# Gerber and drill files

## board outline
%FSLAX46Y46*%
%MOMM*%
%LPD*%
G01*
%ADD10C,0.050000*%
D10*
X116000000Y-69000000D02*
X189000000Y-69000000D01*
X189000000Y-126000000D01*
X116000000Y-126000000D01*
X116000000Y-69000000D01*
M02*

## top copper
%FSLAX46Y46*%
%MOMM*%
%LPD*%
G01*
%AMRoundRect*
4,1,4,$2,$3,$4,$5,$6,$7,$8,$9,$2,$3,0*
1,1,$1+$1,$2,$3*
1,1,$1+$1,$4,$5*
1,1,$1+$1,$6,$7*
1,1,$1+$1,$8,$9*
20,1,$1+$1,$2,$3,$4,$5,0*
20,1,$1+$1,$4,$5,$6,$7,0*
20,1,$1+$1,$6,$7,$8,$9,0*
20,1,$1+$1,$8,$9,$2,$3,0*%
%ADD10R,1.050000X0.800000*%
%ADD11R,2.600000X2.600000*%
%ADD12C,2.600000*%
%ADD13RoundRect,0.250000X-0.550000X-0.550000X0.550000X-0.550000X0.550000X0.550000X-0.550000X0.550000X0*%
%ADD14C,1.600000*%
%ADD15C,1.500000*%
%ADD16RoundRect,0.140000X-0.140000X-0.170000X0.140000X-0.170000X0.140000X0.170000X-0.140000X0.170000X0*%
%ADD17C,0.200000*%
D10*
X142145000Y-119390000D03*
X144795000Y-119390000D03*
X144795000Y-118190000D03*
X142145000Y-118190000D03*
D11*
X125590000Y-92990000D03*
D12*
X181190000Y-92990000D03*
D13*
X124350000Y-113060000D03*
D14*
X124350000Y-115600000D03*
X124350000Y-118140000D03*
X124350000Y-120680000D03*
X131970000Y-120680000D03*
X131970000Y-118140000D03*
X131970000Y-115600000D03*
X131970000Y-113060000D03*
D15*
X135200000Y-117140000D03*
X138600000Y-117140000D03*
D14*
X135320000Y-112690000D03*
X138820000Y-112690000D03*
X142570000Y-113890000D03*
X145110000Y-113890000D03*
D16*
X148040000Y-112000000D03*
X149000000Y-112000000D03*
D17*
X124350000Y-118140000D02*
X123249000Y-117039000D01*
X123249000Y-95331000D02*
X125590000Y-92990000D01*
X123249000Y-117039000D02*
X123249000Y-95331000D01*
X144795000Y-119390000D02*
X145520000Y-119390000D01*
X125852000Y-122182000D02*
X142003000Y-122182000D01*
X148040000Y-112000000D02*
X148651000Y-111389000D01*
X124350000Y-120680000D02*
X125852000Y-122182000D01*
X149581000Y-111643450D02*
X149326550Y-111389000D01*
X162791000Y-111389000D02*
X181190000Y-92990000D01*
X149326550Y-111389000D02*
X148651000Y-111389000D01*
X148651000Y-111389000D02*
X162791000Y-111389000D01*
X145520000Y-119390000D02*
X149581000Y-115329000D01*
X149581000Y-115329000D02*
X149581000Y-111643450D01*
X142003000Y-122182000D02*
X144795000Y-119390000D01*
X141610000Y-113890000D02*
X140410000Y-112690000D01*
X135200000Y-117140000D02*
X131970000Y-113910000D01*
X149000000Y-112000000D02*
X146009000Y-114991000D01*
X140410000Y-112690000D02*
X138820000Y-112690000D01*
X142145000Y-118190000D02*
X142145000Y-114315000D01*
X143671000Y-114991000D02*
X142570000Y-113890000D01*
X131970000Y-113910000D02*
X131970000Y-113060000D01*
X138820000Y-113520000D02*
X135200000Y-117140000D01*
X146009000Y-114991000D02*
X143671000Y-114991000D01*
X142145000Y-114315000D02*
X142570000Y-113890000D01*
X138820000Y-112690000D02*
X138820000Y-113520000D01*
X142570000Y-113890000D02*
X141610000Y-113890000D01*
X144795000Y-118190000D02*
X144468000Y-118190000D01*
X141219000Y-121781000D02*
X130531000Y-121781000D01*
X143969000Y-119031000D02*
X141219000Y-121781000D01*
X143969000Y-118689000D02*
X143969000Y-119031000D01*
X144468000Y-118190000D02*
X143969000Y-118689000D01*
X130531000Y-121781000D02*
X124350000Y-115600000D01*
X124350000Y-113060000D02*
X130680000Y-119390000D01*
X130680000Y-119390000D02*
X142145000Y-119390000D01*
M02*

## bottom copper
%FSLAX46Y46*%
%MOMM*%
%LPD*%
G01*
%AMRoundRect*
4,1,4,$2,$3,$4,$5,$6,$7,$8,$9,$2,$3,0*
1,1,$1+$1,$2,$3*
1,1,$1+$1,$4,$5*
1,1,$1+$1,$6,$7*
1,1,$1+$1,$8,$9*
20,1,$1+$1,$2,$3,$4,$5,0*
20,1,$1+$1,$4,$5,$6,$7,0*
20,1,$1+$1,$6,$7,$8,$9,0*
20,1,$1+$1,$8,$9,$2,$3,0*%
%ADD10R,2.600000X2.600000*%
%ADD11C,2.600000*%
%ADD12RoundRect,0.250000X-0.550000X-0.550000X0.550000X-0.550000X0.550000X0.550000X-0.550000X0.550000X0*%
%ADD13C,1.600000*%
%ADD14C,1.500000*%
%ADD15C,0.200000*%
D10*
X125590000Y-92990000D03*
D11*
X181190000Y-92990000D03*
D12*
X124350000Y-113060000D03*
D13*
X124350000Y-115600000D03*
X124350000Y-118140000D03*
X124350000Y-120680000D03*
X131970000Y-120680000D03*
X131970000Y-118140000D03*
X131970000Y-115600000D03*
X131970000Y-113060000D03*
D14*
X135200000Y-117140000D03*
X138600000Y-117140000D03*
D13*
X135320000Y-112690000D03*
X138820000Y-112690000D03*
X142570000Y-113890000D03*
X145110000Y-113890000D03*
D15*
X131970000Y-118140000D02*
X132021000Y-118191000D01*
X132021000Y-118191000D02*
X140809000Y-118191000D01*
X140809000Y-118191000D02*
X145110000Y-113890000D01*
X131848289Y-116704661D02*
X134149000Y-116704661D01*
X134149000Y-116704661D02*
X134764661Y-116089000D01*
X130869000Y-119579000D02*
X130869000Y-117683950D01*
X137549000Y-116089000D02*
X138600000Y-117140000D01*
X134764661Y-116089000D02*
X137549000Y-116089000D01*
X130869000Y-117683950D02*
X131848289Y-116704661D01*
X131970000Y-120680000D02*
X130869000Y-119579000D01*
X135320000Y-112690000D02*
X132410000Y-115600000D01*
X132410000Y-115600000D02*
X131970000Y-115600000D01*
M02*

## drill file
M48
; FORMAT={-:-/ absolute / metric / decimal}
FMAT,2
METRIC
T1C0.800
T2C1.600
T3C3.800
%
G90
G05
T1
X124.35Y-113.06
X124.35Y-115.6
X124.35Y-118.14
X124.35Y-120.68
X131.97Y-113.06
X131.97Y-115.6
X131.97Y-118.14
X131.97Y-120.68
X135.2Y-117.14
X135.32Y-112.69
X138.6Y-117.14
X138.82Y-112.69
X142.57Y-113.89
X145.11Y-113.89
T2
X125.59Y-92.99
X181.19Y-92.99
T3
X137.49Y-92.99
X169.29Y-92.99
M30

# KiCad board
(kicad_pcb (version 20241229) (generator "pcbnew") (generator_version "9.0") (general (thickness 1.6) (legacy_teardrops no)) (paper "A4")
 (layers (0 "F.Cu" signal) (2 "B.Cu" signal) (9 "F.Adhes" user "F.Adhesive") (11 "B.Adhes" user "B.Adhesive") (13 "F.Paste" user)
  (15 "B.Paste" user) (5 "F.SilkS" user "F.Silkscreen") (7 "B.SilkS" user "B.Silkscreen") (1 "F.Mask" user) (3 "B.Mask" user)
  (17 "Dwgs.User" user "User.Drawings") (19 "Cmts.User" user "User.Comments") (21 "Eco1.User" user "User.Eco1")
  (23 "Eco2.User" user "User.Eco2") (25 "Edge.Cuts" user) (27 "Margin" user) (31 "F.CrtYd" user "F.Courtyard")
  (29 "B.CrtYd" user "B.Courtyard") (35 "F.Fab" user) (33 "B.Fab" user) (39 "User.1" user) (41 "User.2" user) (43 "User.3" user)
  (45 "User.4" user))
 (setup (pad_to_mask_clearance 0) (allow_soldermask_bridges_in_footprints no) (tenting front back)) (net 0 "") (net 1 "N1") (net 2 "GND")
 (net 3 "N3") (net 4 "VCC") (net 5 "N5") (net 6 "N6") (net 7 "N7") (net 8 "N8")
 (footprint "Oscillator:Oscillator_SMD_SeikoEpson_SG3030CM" (layer "F.Cu") (at 143.47 118.79)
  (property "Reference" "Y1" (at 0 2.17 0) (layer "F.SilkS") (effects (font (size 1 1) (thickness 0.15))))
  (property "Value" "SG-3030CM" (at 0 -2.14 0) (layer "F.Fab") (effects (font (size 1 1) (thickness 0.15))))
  (pad "1" smd rect (at -1.325 0.6) (size 1.05 0.8) (layers "F.Cu" "F.Mask" "F.Paste") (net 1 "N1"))
  (pad "2" smd rect (at 1.325 0.6) (size 1.05 0.8) (layers "F.Cu" "F.Mask" "F.Paste") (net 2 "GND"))
  (pad "3" smd rect (at 1.325 -0.6) (size 1.05 0.8) (layers "F.Cu" "F.Mask" "F.Paste") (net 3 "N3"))
  (pad "4" smd rect (at -1.325 -0.6) (size 1.05 0.8) (layers "F.Cu" "F.Mask" "F.Paste") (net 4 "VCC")))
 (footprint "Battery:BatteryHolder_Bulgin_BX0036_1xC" (layer "F.Cu") (at 125.59 92.99)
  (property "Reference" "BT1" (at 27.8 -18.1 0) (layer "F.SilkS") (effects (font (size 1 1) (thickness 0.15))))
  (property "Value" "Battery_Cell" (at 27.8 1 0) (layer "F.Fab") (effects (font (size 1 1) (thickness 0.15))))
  (pad "" np_thru_hole circle (at 11.9 0) (size 3.8 3.8) (drill 3.8) (layers "*.Cu" "*.Mask"))
  (pad "" np_thru_hole circle (at 43.7 0) (size 3.8 3.8) (drill 3.8) (layers "*.Cu" "*.Mask"))
  (pad "1" thru_hole rect (at 0 0) (size 2.6 2.6) (drill 1.6) (layers "*.Cu" "*.Mask") (remove_unused_layers no) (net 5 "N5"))
  (pad "2" thru_hole circle (at 55.6 0) (size 2.6 2.6) (drill 1.6) (layers "*.Cu" "*.Mask") (remove_unused_layers no) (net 2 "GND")))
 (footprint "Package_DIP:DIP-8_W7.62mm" (layer "F.Cu") (at 124.35 113.06)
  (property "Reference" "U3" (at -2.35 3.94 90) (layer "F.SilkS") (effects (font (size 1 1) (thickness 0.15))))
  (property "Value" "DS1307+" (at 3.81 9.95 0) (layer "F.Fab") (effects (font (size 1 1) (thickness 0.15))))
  (pad "1" thru_hole roundrect (at 0 0) (size 1.6 1.6) (drill 0.8) (layers "*.Cu" "*.Mask") (remove_unused_layers no)
   (roundrect_rratio 0.15625) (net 1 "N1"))
  (pad "2" thru_hole circle (at 0 2.54) (size 1.6 1.6) (drill 0.8) (layers "*.Cu" "*.Mask") (remove_unused_layers no) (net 3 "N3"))
  (pad "3" thru_hole circle (at 0 5.08) (size 1.6 1.6) (drill 0.8) (layers "*.Cu" "*.Mask") (remove_unused_layers no) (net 5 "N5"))
  (pad "4" thru_hole circle (at 0 7.62) (size 1.6 1.6) (drill 0.8) (layers "*.Cu" "*.Mask") (remove_unused_layers no) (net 2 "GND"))
  (pad "5" thru_hole circle (at 7.62 7.62) (size 1.6 1.6) (drill 0.8) (layers "*.Cu" "*.Mask") (remove_unused_layers no) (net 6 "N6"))
  (pad "6" thru_hole circle (at 7.62 5.08) (size 1.6 1.6) (drill 0.8) (layers "*.Cu" "*.Mask") (remove_unused_layers no) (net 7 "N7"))
  (pad "7" thru_hole circle (at 7.62 2.54) (size 1.6 1.6) (drill 0.8) (layers "*.Cu" "*.Mask") (remove_unused_layers no) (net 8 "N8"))
  (pad "8" thru_hole circle (at 7.62 0) (size 1.6 1.6) (drill 0.8) (layers "*.Cu" "*.Mask") (remove_unused_layers no) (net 4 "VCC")))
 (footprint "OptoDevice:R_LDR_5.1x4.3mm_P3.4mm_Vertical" (layer "F.Cu") (at 135.2 117.14)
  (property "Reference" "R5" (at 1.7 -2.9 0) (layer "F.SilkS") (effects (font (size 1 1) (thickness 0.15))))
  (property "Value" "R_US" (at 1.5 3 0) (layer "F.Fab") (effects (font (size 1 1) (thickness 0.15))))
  (pad "1" thru_hole circle (at 0 0) (size 1.5 1.5) (drill 0.8) (layers "*.Cu" "*.Mask") (remove_unused_layers no) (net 4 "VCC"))
  (pad "2" thru_hole circle (at 3.4 0) (size 1.5 1.5) (drill 0.8) (layers "*.Cu" "*.Mask") (remove_unused_layers no) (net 6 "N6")))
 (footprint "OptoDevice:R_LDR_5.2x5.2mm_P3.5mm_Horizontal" (layer "F.Cu") (at 135.32 112.69)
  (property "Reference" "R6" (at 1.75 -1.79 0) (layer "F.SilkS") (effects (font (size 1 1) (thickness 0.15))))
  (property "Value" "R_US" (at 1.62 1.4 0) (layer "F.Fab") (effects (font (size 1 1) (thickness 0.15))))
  (pad "1" thru_hole circle (at 0 0) (size 1.6 1.6) (drill 0.8) (layers "*.Cu" "*.Mask") (remove_unused_layers no) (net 8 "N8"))
  (pad "2" thru_hole circle (at 3.5 0) (size 1.6 1.6) (drill 0.8) (layers "*.Cu" "*.Mask") (remove_unused_layers no) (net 4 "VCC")))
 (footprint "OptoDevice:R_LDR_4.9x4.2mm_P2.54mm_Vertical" (layer "F.Cu") (at 142.57 113.89)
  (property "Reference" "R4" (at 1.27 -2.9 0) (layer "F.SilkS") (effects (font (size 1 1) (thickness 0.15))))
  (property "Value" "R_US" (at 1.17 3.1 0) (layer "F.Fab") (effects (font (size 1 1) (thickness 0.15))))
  (pad "1" thru_hole circle (at 0 0) (size 1.6 1.6) (drill 0.8) (layers "*.Cu" "*.Mask") (remove_unused_layers no) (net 4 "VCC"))
  (pad "2" thru_hole circle (at 2.54 0) (size 1.6 1.6) (drill 0.8) (layers "*.Cu" "*.Mask") (remove_unused_layers no) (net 7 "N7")))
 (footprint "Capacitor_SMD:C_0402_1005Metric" (layer "F.Cu") (at 148.52 112)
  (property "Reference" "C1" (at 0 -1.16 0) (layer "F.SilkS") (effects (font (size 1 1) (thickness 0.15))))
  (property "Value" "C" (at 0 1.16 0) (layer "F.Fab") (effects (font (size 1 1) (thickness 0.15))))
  (pad "1" smd roundrect (at -0.48 0) (size 0.56 0.62) (layers "F.Cu" "F.Mask" "F.Paste") (roundrect_rratio 0.25) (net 2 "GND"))
  (pad "2" smd roundrect (at 0.48 0) (size 0.56 0.62) (layers "F.Cu" "F.Mask" "F.Paste") (roundrect_rratio 0.25) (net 4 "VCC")))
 (gr_rect (start 116 69) (end 189 126) (stroke (width 0.05) (type default)) (fill no) (layer "Edge.Cuts"))
 (segment (start 124.35 118.14) (end 123.249 117.039) (width 0.2) (layer "F.Cu") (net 5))
 (segment (start 123.249 95.331) (end 125.59 92.99) (width 0.2) (layer "F.Cu") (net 5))
 (segment (start 123.249 117.039) (end 123.249 95.331) (width 0.2) (layer "F.Cu") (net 5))
 (segment (start 144.795 119.39) (end 145.52 119.39) (width 0.2) (layer "F.Cu") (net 2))
 (segment (start 125.852 122.182) (end 142.003 122.182) (width 0.2) (layer "F.Cu") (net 2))
 (segment (start 148.04 112) (end 148.651 111.389) (width 0.2) (layer "F.Cu") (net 2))
 (segment (start 124.35 120.68) (end 125.852 122.182) (width 0.2) (layer "F.Cu") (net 2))
 (segment (start 149.581 111.64345) (end 149.32655 111.389) (width 0.2) (layer "F.Cu") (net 2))
 (segment (start 162.791 111.389) (end 181.19 92.99) (width 0.2) (layer "F.Cu") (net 2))
 (segment (start 149.32655 111.389) (end 148.651 111.389) (width 0.2) (layer "F.Cu") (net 2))
 (segment (start 148.651 111.389) (end 162.791 111.389) (width 0.2) (layer "F.Cu") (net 2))
 (segment (start 145.52 119.39) (end 149.581 115.329) (width 0.2) (layer "F.Cu") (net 2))
 (segment (start 149.581 115.329) (end 149.581 111.64345) (width 0.2) (layer "F.Cu") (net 2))
 (segment (start 142.003 122.182) (end 144.795 119.39) (width 0.2) (layer "F.Cu") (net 2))
 (segment (start 141.61 113.89) (end 140.41 112.69) (width 0.2) (layer "F.Cu") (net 4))
 (segment (start 135.2 117.14) (end 131.97 113.91) (width 0.2) (layer "F.Cu") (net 4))
 (segment (start 149 112) (end 146.009 114.991) (width 0.2) (layer "F.Cu") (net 4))
 (segment (start 140.41 112.69) (end 138.82 112.69) (width 0.2) (layer "F.Cu") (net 4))
 (segment (start 142.145 118.19) (end 142.145 114.315) (width 0.2) (layer "F.Cu") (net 4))
 (segment (start 143.671 114.991) (end 142.57 113.89) (width 0.2) (layer "F.Cu") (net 4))
 (segment (start 131.97 113.91) (end 131.97 113.06) (width 0.2) (layer "F.Cu") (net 4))
 (segment (start 138.82 113.52) (end 135.2 117.14) (width 0.2) (layer "F.Cu") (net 4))
 (segment (start 146.009 114.991) (end 143.671 114.991) (width 0.2) (layer "F.Cu") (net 4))
 (segment (start 142.145 114.315) (end 142.57 113.89) (width 0.2) (layer "F.Cu") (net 4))
 (segment (start 138.82 112.69) (end 138.82 113.52) (width 0.2) (layer "F.Cu") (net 4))
 (segment (start 142.57 113.89) (end 141.61 113.89) (width 0.2) (layer "F.Cu") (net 4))
 (segment (start 131.97 118.14) (end 132.021 118.191) (width 0.2) (layer "B.Cu") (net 7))
 (segment (start 132.021 118.191) (end 140.809 118.191) (width 0.2) (layer "B.Cu") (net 7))
 (segment (start 140.809 118.191) (end 145.11 113.89) (width 0.2) (layer "B.Cu") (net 7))
 (segment (start 131.848289 116.704661) (end 134.149 116.704661) (width 0.2) (layer "B.Cu") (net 6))
 (segment (start 134.149 116.704661) (end 134.764661 116.089) (width 0.2) (layer "B.Cu") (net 6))
 (segment (start 130.869 119.579) (end 130.869 117.68395) (width 0.2) (layer "B.Cu") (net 6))
 (segment (start 137.549 116.089) (end 138.6 117.14) (width 0.2) (layer "B.Cu") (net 6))
 (segment (start 134.764661 116.089) (end 137.549 116.089) (width 0.2) (layer "B.Cu") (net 6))
 (segment (start 130.869 117.68395) (end 131.848289 116.704661) (width 0.2) (layer "B.Cu") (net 6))
 (segment (start 131.97 120.68) (end 130.869 119.579) (width 0.2) (layer "B.Cu") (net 6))
 (segment (start 135.32 112.69) (end 132.41 115.6) (width 0.2) (layer "B.Cu") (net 8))
 (segment (start 132.41 115.6) (end 131.97 115.6) (width 0.2) (layer "B.Cu") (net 8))
 (segment (start 144.795 118.19) (end 144.468 118.19) (width 0.2) (layer "F.Cu") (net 3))
 (segment (start 141.219 121.781) (end 130.531 121.781) (width 0.2) (layer "F.Cu") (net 3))
 (segment (start 143.969 119.031) (end 141.219 121.781) (width 0.2) (layer "F.Cu") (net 3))
 (segment (start 143.969 118.689) (end 143.969 119.031) (width 0.2) (layer "F.Cu") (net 3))
 (segment (start 144.468 118.19) (end 143.969 118.689) (width 0.2) (layer "F.Cu") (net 3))
 (segment (start 130.531 121.781) (end 124.35 115.6) (width 0.2) (layer "F.Cu") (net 3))
 (segment (start 124.35 113.06) (end 130.68 119.39) (width 0.2) (layer "F.Cu") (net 1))
 (segment (start 130.68 119.39) (end 142.145 119.39) (width 0.2) (layer "F.Cu") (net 1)))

